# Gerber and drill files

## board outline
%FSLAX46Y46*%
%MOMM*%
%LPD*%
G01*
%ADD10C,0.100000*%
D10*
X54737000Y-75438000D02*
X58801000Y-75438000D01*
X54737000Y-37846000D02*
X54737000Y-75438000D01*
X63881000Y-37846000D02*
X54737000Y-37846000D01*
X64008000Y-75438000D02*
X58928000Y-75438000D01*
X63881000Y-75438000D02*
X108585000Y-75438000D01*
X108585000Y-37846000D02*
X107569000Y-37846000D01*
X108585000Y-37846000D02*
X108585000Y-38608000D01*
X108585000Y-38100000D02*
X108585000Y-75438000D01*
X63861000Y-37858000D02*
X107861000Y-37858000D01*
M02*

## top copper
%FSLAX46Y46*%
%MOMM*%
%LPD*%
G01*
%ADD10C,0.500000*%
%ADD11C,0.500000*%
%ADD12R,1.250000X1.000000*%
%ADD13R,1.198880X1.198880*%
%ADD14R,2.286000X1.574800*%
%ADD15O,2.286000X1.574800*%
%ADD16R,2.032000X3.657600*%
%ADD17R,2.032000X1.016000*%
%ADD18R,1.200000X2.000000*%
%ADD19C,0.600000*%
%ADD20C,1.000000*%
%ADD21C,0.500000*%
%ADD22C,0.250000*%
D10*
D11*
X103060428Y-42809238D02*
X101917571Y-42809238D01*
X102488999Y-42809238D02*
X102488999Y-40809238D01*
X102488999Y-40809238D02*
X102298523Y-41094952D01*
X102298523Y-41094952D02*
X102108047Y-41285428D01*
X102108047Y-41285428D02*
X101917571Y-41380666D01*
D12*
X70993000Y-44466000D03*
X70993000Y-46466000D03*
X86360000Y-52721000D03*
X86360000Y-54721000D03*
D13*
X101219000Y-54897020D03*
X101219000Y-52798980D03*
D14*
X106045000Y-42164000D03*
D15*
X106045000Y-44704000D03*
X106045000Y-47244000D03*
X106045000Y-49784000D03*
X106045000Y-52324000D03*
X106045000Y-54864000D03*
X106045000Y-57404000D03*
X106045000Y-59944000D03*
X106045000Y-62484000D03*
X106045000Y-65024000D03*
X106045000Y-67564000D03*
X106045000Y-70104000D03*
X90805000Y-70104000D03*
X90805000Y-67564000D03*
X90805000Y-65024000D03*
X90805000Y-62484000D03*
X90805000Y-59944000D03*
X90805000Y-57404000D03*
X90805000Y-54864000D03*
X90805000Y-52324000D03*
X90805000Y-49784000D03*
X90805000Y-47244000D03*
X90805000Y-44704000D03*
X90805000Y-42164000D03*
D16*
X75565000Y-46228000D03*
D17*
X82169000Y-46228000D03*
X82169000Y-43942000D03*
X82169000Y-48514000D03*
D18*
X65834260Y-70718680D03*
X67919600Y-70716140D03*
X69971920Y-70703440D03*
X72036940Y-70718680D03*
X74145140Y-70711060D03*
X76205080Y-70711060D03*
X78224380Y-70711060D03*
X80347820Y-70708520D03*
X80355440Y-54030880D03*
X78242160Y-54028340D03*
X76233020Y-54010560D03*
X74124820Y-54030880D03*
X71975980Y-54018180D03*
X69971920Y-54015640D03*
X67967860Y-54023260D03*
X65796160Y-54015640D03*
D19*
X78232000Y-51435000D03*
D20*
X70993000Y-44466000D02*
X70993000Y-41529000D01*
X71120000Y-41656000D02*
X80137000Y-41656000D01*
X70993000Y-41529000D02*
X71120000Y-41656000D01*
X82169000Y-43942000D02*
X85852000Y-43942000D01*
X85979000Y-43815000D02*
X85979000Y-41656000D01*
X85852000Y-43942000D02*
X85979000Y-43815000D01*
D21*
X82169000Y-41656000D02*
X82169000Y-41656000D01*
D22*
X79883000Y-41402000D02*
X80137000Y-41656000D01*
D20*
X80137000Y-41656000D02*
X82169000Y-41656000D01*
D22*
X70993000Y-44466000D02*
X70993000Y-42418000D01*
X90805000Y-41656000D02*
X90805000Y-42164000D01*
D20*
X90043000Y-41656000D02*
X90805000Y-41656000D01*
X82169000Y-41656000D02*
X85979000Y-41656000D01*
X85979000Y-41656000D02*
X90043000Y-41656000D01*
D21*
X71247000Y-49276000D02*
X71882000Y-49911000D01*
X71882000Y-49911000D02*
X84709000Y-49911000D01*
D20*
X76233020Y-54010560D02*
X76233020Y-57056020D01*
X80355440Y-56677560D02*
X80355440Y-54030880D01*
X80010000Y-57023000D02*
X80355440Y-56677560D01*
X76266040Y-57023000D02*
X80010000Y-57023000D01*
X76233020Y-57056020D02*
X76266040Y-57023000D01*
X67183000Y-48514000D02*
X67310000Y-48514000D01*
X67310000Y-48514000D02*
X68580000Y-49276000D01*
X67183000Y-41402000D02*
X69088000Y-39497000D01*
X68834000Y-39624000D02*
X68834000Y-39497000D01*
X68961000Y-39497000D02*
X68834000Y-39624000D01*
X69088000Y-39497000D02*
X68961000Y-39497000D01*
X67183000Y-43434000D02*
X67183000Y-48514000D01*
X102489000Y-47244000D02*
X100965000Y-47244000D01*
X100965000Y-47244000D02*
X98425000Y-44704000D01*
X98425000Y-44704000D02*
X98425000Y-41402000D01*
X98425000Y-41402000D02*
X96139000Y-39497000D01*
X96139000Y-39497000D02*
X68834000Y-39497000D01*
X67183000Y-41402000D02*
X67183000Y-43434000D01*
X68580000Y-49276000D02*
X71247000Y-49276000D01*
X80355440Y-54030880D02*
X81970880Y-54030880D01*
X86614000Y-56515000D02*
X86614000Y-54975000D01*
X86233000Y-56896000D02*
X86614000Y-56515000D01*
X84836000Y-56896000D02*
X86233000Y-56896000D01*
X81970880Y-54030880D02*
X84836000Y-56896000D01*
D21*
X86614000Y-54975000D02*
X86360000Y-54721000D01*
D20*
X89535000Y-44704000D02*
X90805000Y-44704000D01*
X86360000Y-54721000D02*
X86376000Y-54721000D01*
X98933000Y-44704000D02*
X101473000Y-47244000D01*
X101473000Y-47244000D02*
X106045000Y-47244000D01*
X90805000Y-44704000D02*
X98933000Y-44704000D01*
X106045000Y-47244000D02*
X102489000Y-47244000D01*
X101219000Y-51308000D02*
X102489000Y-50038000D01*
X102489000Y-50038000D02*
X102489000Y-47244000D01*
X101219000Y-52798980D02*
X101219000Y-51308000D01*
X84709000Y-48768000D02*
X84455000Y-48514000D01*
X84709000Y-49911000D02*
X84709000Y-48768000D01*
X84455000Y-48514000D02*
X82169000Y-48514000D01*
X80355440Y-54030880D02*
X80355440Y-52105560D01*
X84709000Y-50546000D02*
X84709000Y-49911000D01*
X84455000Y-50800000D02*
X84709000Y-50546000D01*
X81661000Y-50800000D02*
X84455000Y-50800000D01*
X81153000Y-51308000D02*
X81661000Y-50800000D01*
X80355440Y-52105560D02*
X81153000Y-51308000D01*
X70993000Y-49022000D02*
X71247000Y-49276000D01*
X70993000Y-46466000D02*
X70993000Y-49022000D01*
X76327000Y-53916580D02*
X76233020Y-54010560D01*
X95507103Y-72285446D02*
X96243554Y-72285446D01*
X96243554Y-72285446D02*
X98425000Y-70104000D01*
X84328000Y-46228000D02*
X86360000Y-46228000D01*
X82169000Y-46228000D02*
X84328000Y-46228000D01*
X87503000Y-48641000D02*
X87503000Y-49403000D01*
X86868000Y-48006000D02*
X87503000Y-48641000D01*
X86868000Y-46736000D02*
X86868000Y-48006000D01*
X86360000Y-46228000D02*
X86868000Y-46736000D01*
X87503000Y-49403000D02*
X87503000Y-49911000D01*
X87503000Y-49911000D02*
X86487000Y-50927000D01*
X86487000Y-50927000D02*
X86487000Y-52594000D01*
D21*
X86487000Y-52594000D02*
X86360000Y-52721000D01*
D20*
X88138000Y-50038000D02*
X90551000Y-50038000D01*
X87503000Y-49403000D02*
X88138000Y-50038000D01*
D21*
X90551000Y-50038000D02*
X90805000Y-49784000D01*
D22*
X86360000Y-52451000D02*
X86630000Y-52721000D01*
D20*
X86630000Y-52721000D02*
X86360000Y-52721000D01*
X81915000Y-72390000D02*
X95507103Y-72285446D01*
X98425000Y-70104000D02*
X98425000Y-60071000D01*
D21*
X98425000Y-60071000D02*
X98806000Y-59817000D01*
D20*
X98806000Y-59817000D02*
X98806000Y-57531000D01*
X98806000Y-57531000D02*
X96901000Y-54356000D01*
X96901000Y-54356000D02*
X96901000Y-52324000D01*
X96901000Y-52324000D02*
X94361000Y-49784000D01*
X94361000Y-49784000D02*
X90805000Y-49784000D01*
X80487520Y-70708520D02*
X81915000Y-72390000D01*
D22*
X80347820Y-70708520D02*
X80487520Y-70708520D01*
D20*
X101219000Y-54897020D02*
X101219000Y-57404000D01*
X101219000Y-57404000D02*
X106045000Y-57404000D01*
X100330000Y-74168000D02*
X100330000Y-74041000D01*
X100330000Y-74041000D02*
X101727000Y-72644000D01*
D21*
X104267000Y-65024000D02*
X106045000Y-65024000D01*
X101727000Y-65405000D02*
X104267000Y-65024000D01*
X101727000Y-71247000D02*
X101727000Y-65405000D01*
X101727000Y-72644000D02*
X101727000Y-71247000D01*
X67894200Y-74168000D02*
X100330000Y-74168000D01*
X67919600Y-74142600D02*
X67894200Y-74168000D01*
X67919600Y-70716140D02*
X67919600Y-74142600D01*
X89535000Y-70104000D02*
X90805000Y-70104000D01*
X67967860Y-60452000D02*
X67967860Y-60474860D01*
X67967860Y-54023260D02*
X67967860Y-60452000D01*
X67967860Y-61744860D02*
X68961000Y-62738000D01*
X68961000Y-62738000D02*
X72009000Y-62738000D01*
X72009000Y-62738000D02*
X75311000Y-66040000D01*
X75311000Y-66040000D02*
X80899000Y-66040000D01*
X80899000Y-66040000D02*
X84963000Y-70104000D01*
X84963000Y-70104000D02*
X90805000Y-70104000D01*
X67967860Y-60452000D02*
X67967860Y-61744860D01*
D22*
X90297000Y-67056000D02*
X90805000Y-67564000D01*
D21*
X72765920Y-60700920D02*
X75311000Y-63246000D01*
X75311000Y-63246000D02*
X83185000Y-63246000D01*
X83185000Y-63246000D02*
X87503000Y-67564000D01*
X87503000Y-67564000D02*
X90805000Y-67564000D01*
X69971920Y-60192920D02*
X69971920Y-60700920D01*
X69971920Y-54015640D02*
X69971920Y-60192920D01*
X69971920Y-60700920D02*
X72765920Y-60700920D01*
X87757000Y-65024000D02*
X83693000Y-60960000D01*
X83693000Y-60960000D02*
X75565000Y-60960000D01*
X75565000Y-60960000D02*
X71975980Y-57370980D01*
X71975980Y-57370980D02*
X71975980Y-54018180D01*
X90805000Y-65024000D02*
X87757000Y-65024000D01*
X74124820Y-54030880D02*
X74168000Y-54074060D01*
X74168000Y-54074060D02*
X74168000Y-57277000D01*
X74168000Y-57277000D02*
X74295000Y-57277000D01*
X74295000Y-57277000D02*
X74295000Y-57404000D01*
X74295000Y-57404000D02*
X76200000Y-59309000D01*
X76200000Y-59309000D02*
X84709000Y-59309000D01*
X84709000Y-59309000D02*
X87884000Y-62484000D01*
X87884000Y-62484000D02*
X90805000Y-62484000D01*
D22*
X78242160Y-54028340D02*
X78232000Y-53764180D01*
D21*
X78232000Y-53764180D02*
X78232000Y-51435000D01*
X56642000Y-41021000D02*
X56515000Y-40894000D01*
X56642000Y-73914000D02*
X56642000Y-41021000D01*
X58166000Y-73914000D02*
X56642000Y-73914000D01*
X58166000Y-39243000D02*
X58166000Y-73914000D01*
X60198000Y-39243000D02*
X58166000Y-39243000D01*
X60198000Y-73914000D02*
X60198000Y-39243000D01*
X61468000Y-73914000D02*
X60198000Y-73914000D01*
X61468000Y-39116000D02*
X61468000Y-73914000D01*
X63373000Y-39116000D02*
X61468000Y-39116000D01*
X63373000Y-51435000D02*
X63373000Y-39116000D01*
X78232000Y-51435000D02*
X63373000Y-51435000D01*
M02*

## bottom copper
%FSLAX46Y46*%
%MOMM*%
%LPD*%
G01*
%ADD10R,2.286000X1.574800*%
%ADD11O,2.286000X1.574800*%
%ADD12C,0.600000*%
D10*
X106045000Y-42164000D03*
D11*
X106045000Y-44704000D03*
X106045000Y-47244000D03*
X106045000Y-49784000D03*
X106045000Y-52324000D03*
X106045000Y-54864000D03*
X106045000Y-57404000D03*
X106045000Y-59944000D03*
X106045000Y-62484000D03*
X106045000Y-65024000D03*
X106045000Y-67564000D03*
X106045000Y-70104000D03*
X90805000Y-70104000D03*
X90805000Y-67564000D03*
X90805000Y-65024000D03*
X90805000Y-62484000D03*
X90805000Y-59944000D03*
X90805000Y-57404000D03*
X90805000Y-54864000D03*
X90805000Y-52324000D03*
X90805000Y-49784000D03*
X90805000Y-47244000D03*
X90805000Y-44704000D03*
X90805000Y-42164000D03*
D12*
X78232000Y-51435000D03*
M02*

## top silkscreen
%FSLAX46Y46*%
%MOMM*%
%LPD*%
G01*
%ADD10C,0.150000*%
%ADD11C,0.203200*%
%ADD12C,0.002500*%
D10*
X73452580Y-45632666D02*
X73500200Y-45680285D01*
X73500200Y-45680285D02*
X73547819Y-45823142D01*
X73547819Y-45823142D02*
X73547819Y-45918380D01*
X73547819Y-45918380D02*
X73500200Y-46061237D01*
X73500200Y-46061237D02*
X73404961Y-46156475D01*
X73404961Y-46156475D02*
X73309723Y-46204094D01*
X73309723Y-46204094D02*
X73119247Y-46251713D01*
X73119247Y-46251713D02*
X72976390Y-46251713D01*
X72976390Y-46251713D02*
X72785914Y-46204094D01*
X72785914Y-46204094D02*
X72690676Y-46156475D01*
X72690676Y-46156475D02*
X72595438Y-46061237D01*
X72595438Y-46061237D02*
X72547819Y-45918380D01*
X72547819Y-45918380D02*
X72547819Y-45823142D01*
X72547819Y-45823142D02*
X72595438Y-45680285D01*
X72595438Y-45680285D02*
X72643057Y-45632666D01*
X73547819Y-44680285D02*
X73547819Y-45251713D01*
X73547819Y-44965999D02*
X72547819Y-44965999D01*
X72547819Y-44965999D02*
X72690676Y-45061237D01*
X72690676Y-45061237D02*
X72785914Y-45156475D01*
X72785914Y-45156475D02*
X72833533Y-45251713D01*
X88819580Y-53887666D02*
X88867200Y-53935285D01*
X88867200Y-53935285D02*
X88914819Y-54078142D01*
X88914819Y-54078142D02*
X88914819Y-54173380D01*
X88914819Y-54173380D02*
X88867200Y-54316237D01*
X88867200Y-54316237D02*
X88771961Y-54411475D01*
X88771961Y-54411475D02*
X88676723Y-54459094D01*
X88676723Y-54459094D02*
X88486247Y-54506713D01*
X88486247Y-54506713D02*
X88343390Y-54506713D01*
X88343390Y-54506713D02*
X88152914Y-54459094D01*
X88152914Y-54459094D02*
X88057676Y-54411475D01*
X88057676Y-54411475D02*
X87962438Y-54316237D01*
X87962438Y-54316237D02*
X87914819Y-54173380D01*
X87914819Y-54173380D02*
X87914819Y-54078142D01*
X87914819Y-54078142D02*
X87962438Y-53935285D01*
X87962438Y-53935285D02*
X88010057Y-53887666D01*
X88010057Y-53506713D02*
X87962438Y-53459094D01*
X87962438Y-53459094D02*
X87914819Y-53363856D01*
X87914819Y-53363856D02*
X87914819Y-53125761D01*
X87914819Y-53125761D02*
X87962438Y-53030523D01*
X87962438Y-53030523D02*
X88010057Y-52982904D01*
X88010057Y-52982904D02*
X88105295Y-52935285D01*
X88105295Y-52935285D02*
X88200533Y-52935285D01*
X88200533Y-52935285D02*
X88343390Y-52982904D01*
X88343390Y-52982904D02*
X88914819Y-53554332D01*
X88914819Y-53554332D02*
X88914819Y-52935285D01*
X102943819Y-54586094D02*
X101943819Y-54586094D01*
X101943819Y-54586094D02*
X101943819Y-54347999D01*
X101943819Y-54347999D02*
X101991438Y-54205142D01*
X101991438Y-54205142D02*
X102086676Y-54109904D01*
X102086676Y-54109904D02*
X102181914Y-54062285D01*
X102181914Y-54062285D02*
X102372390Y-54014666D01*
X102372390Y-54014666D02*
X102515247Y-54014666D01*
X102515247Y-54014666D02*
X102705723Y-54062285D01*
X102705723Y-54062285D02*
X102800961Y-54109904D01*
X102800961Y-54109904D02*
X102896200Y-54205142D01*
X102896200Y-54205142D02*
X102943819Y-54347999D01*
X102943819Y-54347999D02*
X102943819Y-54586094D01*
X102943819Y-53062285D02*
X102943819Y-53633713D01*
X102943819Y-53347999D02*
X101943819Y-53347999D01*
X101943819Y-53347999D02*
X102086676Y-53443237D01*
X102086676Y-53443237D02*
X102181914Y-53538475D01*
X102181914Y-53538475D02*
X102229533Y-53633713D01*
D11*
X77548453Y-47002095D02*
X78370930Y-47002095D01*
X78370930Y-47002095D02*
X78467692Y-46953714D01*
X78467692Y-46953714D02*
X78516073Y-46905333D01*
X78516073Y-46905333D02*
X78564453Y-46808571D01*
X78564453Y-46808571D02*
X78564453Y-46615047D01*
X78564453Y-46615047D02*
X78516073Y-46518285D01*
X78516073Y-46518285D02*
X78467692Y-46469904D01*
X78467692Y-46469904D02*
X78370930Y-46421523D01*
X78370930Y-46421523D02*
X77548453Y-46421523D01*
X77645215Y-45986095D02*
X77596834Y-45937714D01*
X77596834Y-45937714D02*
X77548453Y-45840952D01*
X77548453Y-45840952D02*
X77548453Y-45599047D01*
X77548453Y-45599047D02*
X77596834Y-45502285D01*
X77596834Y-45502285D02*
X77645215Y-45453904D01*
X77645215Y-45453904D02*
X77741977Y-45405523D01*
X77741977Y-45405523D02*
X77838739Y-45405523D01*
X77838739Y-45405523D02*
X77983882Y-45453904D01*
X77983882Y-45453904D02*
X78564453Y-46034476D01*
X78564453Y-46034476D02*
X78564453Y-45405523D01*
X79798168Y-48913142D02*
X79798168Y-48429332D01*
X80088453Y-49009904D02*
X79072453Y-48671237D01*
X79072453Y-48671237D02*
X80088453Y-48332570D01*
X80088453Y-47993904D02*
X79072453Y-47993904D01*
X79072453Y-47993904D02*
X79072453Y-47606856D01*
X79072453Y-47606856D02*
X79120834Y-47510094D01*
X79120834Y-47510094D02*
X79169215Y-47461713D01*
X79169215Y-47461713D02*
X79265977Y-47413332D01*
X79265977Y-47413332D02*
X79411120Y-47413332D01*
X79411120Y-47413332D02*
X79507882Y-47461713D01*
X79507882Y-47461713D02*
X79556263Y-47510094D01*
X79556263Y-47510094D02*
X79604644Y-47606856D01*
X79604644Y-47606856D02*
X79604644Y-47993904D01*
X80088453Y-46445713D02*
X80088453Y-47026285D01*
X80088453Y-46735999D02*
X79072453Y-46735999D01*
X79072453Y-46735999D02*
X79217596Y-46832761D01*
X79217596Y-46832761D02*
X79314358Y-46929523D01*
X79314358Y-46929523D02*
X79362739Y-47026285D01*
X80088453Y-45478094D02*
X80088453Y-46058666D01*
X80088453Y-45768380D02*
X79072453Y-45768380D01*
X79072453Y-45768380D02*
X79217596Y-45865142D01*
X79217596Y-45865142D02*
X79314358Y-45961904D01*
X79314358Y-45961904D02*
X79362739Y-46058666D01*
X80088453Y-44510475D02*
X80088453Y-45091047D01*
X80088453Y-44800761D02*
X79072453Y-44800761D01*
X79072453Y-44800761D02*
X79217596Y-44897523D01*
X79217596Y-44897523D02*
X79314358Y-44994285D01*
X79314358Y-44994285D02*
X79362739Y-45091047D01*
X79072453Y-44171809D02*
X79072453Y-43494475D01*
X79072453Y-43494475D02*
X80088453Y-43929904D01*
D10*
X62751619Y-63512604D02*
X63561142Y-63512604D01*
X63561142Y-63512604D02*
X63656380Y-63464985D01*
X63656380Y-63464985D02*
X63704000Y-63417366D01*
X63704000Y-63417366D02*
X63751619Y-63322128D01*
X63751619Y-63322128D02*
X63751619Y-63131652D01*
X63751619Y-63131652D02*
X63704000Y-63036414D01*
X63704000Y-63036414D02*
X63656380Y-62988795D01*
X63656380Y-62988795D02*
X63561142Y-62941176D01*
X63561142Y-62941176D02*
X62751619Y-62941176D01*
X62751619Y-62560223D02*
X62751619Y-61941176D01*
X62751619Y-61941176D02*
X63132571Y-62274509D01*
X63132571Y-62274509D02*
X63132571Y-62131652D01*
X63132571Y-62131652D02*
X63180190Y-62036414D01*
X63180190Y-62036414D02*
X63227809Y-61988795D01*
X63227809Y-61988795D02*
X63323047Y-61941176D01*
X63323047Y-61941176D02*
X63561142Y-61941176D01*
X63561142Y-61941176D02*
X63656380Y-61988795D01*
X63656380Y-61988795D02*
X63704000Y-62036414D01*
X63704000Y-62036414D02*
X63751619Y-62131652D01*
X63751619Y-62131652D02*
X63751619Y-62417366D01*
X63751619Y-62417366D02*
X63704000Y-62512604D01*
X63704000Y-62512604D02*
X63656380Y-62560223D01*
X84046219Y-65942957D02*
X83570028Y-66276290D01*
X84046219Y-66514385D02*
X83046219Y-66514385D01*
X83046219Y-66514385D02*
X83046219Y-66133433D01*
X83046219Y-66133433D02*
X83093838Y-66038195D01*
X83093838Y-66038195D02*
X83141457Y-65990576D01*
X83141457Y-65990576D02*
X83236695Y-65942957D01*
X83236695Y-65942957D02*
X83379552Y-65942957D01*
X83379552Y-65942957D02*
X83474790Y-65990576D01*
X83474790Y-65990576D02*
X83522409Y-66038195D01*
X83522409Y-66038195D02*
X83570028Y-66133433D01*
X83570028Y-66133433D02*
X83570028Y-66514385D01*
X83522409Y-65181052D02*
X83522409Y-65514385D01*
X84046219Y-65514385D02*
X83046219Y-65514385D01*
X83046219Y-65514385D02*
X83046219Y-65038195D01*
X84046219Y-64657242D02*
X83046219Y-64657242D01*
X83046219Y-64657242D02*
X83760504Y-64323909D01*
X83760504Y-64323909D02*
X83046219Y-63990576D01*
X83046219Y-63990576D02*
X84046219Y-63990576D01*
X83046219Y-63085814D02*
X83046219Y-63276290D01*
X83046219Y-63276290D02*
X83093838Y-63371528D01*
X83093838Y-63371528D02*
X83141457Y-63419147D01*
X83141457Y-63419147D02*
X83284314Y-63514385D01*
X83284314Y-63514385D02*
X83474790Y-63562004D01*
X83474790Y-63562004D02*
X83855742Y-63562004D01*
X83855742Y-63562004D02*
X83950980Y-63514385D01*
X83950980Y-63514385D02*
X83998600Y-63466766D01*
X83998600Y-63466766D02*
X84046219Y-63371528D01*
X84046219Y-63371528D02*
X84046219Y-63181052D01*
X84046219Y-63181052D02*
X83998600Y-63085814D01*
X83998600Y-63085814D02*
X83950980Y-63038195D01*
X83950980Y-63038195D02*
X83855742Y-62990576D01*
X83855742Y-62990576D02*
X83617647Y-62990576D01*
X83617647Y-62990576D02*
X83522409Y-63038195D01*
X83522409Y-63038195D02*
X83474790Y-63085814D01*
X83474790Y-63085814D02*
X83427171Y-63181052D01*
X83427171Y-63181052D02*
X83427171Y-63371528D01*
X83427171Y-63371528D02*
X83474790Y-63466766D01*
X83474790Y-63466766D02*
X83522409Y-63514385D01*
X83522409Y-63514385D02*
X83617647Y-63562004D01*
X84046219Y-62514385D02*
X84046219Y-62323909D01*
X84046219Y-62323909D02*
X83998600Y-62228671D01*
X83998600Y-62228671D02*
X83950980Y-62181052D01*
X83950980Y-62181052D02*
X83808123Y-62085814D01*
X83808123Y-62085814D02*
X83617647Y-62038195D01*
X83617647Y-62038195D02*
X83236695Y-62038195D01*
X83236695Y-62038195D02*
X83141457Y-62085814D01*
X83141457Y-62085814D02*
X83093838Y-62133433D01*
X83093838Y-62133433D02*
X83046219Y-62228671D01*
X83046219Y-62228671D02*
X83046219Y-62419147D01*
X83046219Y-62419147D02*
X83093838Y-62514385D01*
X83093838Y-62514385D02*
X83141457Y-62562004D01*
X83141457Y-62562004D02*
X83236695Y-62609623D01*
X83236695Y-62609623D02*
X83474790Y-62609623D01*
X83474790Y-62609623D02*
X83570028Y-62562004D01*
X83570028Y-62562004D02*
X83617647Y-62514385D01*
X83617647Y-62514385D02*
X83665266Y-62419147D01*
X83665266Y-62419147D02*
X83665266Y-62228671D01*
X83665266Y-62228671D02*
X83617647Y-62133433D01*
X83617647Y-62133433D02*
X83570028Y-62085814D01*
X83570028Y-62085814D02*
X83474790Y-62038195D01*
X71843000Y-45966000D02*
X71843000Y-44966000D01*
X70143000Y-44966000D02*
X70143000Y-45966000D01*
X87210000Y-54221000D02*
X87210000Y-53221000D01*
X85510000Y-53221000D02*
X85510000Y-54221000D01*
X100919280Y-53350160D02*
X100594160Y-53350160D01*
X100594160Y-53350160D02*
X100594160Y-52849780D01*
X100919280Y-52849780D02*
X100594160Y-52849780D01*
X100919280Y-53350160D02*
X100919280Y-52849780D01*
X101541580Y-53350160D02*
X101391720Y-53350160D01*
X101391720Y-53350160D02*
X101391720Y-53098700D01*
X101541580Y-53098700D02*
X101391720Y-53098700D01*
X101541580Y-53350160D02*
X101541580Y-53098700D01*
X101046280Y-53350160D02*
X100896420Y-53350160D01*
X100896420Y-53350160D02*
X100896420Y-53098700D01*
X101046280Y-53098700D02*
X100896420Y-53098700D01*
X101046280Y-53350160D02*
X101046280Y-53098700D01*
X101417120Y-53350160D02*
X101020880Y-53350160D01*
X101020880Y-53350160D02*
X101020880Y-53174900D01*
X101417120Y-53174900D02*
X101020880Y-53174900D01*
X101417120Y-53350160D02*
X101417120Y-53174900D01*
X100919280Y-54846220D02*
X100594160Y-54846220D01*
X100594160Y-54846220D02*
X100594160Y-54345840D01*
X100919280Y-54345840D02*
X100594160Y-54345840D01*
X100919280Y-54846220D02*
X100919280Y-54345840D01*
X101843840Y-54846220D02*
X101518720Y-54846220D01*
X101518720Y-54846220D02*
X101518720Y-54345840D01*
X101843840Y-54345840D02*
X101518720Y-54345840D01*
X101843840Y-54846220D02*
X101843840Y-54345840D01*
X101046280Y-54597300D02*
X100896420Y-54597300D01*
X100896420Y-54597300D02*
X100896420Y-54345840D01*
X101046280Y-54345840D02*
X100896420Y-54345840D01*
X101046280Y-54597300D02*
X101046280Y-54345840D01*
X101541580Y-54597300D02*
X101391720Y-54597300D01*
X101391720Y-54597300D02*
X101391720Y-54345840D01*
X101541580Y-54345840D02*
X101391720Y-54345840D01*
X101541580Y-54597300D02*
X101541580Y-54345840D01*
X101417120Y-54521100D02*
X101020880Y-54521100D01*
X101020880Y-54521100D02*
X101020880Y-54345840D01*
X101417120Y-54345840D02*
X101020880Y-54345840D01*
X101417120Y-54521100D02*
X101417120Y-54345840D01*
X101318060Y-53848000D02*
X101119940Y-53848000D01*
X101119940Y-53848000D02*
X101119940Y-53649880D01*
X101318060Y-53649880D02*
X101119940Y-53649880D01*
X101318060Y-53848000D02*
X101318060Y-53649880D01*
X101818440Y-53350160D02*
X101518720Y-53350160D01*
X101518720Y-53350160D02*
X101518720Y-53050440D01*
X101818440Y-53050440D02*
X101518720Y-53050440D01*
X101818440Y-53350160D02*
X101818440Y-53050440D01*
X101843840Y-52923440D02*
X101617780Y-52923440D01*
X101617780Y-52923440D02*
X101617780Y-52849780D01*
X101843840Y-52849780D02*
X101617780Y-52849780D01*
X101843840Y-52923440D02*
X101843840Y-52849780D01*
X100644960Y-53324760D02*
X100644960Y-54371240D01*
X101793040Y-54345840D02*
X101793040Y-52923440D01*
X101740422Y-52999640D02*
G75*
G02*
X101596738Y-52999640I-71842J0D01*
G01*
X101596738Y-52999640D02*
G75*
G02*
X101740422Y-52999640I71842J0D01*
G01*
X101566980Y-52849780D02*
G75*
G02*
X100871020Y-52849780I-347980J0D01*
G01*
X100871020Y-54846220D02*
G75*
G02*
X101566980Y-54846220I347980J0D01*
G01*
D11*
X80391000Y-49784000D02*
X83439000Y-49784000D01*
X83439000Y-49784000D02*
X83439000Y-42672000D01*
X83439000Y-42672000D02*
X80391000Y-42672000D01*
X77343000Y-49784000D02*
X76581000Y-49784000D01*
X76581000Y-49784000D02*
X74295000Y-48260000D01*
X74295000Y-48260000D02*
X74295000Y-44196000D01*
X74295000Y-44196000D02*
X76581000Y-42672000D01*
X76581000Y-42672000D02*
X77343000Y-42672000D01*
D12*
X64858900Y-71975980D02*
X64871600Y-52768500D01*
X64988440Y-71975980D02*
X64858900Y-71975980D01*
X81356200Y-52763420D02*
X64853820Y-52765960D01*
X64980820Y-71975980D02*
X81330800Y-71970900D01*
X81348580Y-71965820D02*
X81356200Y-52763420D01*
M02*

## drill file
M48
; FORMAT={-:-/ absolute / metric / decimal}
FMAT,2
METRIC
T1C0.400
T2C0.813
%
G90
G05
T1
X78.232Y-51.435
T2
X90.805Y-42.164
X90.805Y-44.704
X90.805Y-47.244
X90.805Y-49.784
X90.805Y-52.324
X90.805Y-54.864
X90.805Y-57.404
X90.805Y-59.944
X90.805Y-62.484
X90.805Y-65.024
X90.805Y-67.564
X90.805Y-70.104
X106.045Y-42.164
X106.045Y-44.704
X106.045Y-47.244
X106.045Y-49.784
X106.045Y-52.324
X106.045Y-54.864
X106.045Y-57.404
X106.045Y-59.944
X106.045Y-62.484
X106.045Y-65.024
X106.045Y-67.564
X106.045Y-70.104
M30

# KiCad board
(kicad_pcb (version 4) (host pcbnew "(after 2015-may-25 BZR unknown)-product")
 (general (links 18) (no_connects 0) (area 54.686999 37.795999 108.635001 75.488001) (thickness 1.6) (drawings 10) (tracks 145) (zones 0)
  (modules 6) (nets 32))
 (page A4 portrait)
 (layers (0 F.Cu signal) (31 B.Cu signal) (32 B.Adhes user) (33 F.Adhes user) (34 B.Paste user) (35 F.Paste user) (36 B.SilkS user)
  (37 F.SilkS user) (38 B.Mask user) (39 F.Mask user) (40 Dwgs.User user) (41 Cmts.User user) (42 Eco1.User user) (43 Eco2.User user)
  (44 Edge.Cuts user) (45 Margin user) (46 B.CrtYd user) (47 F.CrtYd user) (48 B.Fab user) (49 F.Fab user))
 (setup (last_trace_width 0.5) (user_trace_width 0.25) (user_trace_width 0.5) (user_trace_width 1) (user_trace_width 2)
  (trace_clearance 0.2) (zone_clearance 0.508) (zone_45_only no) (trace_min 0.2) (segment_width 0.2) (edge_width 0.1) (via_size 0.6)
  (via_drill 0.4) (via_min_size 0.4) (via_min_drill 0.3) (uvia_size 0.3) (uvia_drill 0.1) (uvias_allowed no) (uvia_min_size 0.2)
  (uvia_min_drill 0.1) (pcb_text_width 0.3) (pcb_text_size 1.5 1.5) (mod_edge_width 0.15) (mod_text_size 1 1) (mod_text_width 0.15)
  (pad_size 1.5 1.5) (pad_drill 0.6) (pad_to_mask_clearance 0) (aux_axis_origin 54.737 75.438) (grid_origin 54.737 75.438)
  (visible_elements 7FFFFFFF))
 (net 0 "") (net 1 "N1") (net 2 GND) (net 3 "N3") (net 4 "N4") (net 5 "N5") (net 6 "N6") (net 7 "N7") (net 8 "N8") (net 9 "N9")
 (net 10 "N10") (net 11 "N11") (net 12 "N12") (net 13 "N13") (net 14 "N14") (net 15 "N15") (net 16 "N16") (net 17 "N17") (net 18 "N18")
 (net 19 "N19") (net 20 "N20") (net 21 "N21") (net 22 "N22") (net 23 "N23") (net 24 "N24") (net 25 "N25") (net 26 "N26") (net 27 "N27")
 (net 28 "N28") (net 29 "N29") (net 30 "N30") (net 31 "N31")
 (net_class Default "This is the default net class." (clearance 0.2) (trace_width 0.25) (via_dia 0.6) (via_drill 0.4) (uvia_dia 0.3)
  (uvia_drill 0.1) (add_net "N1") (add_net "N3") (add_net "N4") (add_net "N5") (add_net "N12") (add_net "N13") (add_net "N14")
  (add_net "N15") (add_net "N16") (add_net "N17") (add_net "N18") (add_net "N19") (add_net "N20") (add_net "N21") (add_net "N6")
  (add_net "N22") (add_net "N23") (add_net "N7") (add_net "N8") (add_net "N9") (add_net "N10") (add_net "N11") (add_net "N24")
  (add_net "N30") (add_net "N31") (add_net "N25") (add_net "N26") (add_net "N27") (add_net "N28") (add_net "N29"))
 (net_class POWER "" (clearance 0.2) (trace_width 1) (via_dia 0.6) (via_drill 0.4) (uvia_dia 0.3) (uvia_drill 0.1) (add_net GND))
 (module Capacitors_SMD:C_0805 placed (layer F.Cu) (at 70.993 45.466 270)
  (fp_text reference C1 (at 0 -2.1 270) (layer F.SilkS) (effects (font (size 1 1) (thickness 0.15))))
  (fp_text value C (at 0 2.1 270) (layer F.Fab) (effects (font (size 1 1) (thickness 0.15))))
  (fp_line (start 0.5 -0.85) (end -0.5 -0.85) (layer F.SilkS) (width 0.15))
  (fp_line (start -0.5 0.85) (end 0.5 0.85) (layer F.SilkS) (width 0.15))
  (pad 1 smd rect (at -1 0 270) (size 1 1.25) (layers F.Cu F.Paste F.Mask) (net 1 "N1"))
  (pad 2 smd rect (at 1 0 270) (size 1 1.25) (layers F.Cu F.Paste F.Mask) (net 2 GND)))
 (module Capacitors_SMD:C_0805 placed (layer F.Cu) (at 86.36 53.721 270)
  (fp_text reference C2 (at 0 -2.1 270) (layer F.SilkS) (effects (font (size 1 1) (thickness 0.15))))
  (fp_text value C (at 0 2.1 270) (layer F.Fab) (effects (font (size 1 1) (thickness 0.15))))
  (fp_line (start 0.5 -0.85) (end -0.5 -0.85) (layer F.SilkS) (width 0.15))
  (fp_line (start -0.5 0.85) (end 0.5 0.85) (layer F.SilkS) (width 0.15))
  (pad 1 smd rect (at -1 0 270) (size 1 1.25) (layers F.Cu F.Paste F.Mask) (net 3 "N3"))
  (pad 2 smd rect (at 1 0 270) (size 1 1.25) (layers F.Cu F.Paste F.Mask) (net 2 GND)))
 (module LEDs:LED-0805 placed (layer F.Cu) (at 101.219 53.848 270)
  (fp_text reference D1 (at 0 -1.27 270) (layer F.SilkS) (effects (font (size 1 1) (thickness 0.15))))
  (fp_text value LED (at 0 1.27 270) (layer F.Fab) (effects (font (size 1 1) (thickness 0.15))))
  (fp_line (start -0.49784 0.29972) (end -0.49784 0.62484) (layer F.SilkS) (width 0.15))
  (fp_line (start -0.49784 0.62484) (end -0.99822 0.62484) (layer F.SilkS) (width 0.15))
  (fp_line (start -0.99822 0.29972) (end -0.99822 0.62484) (layer F.SilkS) (width 0.15))
  (fp_line (start -0.49784 0.29972) (end -0.99822 0.29972) (layer F.SilkS) (width 0.15))
  (fp_line (start -0.49784 -0.32258) (end -0.49784 -0.17272) (layer F.SilkS) (width 0.15))
  (fp_line (start -0.49784 -0.17272) (end -0.7493 -0.17272) (layer F.SilkS) (width 0.15))
  (fp_line (start -0.7493 -0.32258) (end -0.7493 -0.17272) (layer F.SilkS) (width 0.15))
  (fp_line (start -0.49784 -0.32258) (end -0.7493 -0.32258) (layer F.SilkS) (width 0.15))
  (fp_line (start -0.49784 0.17272) (end -0.49784 0.32258) (layer F.SilkS) (width 0.15))
  (fp_line (start -0.49784 0.32258) (end -0.7493 0.32258) (layer F.SilkS) (width 0.15))
  (fp_line (start -0.7493 0.17272) (end -0.7493 0.32258) (layer F.SilkS) (width 0.15))
  (fp_line (start -0.49784 0.17272) (end -0.7493 0.17272) (layer F.SilkS) (width 0.15))
  (fp_line (start -0.49784 -0.19812) (end -0.49784 0.19812) (layer F.SilkS) (width 0.15))
  (fp_line (start -0.49784 0.19812) (end -0.6731 0.19812) (layer F.SilkS) (width 0.15))
  (fp_line (start -0.6731 -0.19812) (end -0.6731 0.19812) (layer F.SilkS) (width 0.15))
  (fp_line (start -0.49784 -0.19812) (end -0.6731 -0.19812) (layer F.SilkS) (width 0.15))
  (fp_line (start 0.99822 0.29972) (end 0.99822 0.62484) (layer F.SilkS) (width 0.15))
  (fp_line (start 0.99822 0.62484) (end 0.49784 0.62484) (layer F.SilkS) (width 0.15))
  (fp_line (start 0.49784 0.29972) (end 0.49784 0.62484) (layer F.SilkS) (width 0.15))
  (fp_line (start 0.99822 0.29972) (end 0.49784 0.29972) (layer F.SilkS) (width 0.15))
  (fp_line (start 0.99822 -0.62484) (end 0.99822 -0.29972) (layer F.SilkS) (width 0.15))
  (fp_line (start 0.99822 -0.29972) (end 0.49784 -0.29972) (layer F.SilkS) (width 0.15))
  (fp_line (start 0.49784 -0.62484) (end 0.49784 -0.29972) (layer F.SilkS) (width 0.15))
  (fp_line (start 0.99822 -0.62484) (end 0.49784 -0.62484) (layer F.SilkS) (width 0.15))
  (fp_line (start 0.7493 0.17272) (end 0.7493 0.32258) (layer F.SilkS) (width 0.15))
  (fp_line (start 0.7493 0.32258) (end 0.49784 0.32258) (layer F.SilkS) (width 0.15))
  (fp_line (start 0.49784 0.17272) (end 0.49784 0.32258) (layer F.SilkS) (width 0.15))
  (fp_line (start 0.7493 0.17272) (end 0.49784 0.17272) (layer F.SilkS) (width 0.15))
  (fp_line (start 0.7493 -0.32258) (end 0.7493 -0.17272) (layer F.SilkS) (width 0.15))
  (fp_line (start 0.7493 -0.17272) (end 0.49784 -0.17272) (layer F.SilkS) (width 0.15))
  (fp_line (start 0.49784 -0.32258) (end 0.49784 -0.17272) (layer F.SilkS) (width 0.15))
  (fp_line (start 0.7493 -0.32258) (end 0.49784 -0.32258) (layer F.SilkS) (width 0.15))
  (fp_line (start 0.6731 -0.19812) (end 0.6731 0.19812) (layer F.SilkS) (width 0.15))
  (fp_line (start 0.6731 0.19812) (end 0.49784 0.19812) (layer F.SilkS) (width 0.15))
  (fp_line (start 0.49784 -0.19812) (end 0.49784 0.19812) (layer F.SilkS) (width 0.15))
  (fp_line (start 0.6731 -0.19812) (end 0.49784 -0.19812) (layer F.SilkS) (width 0.15))
  (fp_line (start 0 -0.09906) (end 0 0.09906) (layer F.SilkS) (width 0.15))
  (fp_line (start 0 0.09906) (end -0.19812 0.09906) (layer F.SilkS) (width 0.15))
  (fp_line (start -0.19812 -0.09906) (end -0.19812 0.09906) (layer F.SilkS) (width 0.15))
  (fp_line (start 0 -0.09906) (end -0.19812 -0.09906) (layer F.SilkS) (width 0.15))
  (fp_line (start -0.49784 -0.59944) (end -0.49784 -0.29972) (layer F.SilkS) (width 0.15))
  (fp_line (start -0.49784 -0.29972) (end -0.79756 -0.29972) (layer F.SilkS) (width 0.15))
  (fp_line (start -0.79756 -0.59944) (end -0.79756 -0.29972) (layer F.SilkS) (width 0.15))
  (fp_line (start -0.49784 -0.59944) (end -0.79756 -0.59944) (layer F.SilkS) (width 0.15))
  (fp_line (start -0.92456 -0.62484) (end -0.92456 -0.39878) (layer F.SilkS) (width 0.15))
  (fp_line (start -0.92456 -0.39878) (end -0.99822 -0.39878) (layer F.SilkS) (width 0.15))
  (fp_line (start -0.99822 -0.62484) (end -0.99822 -0.39878) (layer F.SilkS) (width 0.15))
  (fp_line (start -0.92456 -0.62484) (end -0.99822 -0.62484) (layer F.SilkS) (width 0.15))
  (fp_line (start -0.52324 0.57404) (end 0.52324 0.57404) (layer F.SilkS) (width 0.15))
  (fp_line (start 0.49784 -0.57404) (end -0.92456 -0.57404) (layer F.SilkS) (width 0.15))
  (fp_circle (center -0.84836 -0.44958) (end -0.89916 -0.50038) (layer F.SilkS) (width 0.15))
  (fp_arc (start -0.99822 0) (end -0.99822 0.34798) (angle -180) (layer F.SilkS) (width 0.15))
  (fp_arc (start 0.99822 0) (end 0.99822 -0.34798) (angle -180) (layer F.SilkS) (width 0.15))
  (pad 2 smd rect (at 1.04902 0 90) (size 1.19888 1.19888) (layers F.Cu F.Paste F.Mask) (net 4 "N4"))
  (pad 1 smd rect (at -1.04902 0 90) (size 1.19888 1.19888) (layers F.Cu F.Paste F.Mask) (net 2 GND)))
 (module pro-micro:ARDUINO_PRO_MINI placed (layer B.Cu) (at 102.235 56.134 270)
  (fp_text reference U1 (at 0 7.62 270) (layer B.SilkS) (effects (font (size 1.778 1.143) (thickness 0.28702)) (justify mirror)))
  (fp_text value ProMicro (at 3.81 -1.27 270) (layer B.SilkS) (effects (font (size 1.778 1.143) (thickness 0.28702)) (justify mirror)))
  (pad 1 thru_hole rect (at -13.97 -3.81 270) (size 1.5748 2.286) (drill 0.8128) (layers *.Cu *.Mask B.SilkS) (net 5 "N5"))
  (pad 2 thru_hole oval (at -11.43 -3.81 270) (size 1.5748 2.286) (drill 0.8128) (layers *.Cu *.Mask B.SilkS) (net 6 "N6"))
  (pad 3 thru_hole oval (at -8.89 -3.81 270) (size 1.5748 2.286) (drill 0.8128) (layers *.Cu *.Mask B.SilkS) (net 2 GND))
  (pad 4 thru_hole oval (at -6.35 -3.81 270) (size 1.5748 2.286) (drill 0.8128) (layers *.Cu *.Mask B.SilkS) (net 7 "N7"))
  (pad 5 thru_hole oval (at -3.81 -3.81 270) (size 1.5748 2.286) (drill 0.8128) (layers *.Cu *.Mask B.SilkS) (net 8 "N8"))
  (pad 6 thru_hole oval (at -1.27 -3.81 270) (size 1.5748 2.286) (drill 0.8128) (layers *.Cu *.Mask B.SilkS) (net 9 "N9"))
  (pad 7 thru_hole oval (at 1.27 -3.81 270) (size 1.5748 2.286) (drill 0.8128) (layers *.Cu *.Mask B.SilkS) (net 4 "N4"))
  (pad 8 thru_hole oval (at 3.81 -3.81 270) (size 1.5748 2.286) (drill 0.8128) (layers *.Cu *.Mask B.SilkS) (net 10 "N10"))
  (pad 9 thru_hole oval (at 6.35 -3.81 270) (size 1.5748 2.286) (drill 0.8128) (layers *.Cu *.Mask B.SilkS) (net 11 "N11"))
  (pad 10 thru_hole oval (at 8.89 -3.81 270) (size 1.5748 2.286) (drill 0.8128) (layers *.Cu *.Mask B.SilkS) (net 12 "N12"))
  (pad 11 thru_hole oval (at 11.43 -3.81 270) (size 1.5748 2.286) (drill 0.8128) (layers *.Cu *.Mask B.SilkS) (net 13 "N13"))
  (pad 12 thru_hole oval (at 13.97 -3.81 270) (size 1.5748 2.286) (drill 0.8128) (layers *.Cu *.Mask B.SilkS) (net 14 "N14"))
  (pad 13 thru_hole oval (at 13.97 11.43 270) (size 1.5748 2.286) (drill 0.8128) (layers *.Cu *.Mask B.SilkS) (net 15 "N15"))
  (pad 14 thru_hole oval (at 11.43 11.43 270) (size 1.5748 2.286) (drill 0.8128) (layers *.Cu *.Mask B.SilkS) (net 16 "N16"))
  (pad 15 thru_hole oval (at 8.89 11.43 270) (size 1.5748 2.286) (drill 0.8128) (layers *.Cu *.Mask B.SilkS) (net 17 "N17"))
  (pad 16 thru_hole oval (at 6.35 11.43 270) (size 1.5748 2.286) (drill 0.8128) (layers *.Cu *.Mask B.SilkS) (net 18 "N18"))
  (pad 17 thru_hole oval (at 3.81 11.43 270) (size 1.5748 2.286) (drill 0.8128) (layers *.Cu *.Mask B.SilkS) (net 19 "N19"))
  (pad 18 thru_hole oval (at 1.27 11.43 270) (size 1.5748 2.286) (drill 0.8128) (layers *.Cu *.Mask B.SilkS) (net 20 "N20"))
  (pad 19 thru_hole oval (at -1.27 11.43 270) (size 1.5748 2.286) (drill 0.8128) (layers *.Cu *.Mask B.SilkS) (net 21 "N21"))
  (pad 20 thru_hole oval (at -3.81 11.43 270) (size 1.5748 2.286) (drill 0.8128) (layers *.Cu *.Mask B.SilkS) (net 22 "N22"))
  (pad 21 thru_hole oval (at -6.35 11.43 270) (size 1.5748 2.286) (drill 0.8128) (layers *.Cu *.Mask B.SilkS) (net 3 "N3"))
  (pad 22 thru_hole oval (at -8.89 11.43 270) (size 1.5748 2.286) (drill 0.8128) (layers *.Cu *.Mask B.SilkS) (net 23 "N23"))
  (pad 23 thru_hole oval (at -11.43 11.43 270) (size 1.5748 2.286) (drill 0.8128) (layers *.Cu *.Mask B.SilkS) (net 2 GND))
  (pad 24 thru_hole oval (at -13.97 11.43 270) (size 1.5748 2.286) (drill 0.8128) (layers *.Cu *.Mask B.SilkS) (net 1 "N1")))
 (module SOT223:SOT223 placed (layer F.Cu) (at 78.867 46.228 90)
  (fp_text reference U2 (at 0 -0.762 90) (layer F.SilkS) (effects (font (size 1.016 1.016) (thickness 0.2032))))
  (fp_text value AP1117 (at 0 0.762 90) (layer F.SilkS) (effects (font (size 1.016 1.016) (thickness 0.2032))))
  (fp_line (start -3.556 1.524) (end -3.556 4.572) (layer F.SilkS) (width 0.2032))
  (fp_line (start -3.556 4.572) (end 3.556 4.572) (layer F.SilkS) (width 0.2032))
  (fp_line (start 3.556 4.572) (end 3.556 1.524) (layer F.SilkS) (width 0.2032))
  (fp_line (start -3.556 -1.524) (end -3.556 -2.286) (layer F.SilkS) (width 0.2032))
  (fp_line (start -3.556 -2.286) (end -2.032 -4.572) (layer F.SilkS) (width 0.2032))
  (fp_line (start -2.032 -4.572) (end 2.032 -4.572) (layer F.SilkS) (width 0.2032))
  (fp_line (start 2.032 -4.572) (end 3.556 -2.286) (layer F.SilkS) (width 0.2032))
  (fp_line (start 3.556 -2.286) (end 3.556 -1.524) (layer F.SilkS) (width 0.2032))
  (pad 4 smd rect (at 0 -3.302 90) (size 3.6576 2.032) (layers F.Cu F.Paste F.Mask))
  (pad 2 smd rect (at 0 3.302 90) (size 1.016 2.032) (layers F.Cu F.Paste F.Mask) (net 3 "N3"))
  (pad 3 smd rect (at 2.286 3.302 90) (size 1.016 2.032) (layers F.Cu F.Paste F.Mask) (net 1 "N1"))
  (pad 1 smd rect (at -2.286 3.302 90) (size 1.016 2.032) (layers F.Cu F.Paste F.Mask) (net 2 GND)))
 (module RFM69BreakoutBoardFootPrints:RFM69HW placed (layer F.Cu) (at 74.041 62.738 90)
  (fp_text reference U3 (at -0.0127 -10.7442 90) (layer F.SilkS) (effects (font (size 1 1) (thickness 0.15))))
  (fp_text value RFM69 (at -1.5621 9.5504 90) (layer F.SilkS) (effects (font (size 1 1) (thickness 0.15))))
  (fp_line (start -9.23798 -9.1821) (end 9.9695 -9.1694) (layer F.SilkS) (width 0.0025))
  (fp_line (start -9.23798 -9.05256) (end -9.23798 -9.1821) (layer F.SilkS) (width 0.0025))
  (fp_line (start 9.97458 7.3152) (end 9.97204 -9.18718) (layer F.SilkS) (width 0.0025))
  (fp_line (start -9.23798 -9.06018) (end -9.2329 7.2898) (layer F.SilkS) (width 0.0025))
  (fp_line (start -9.22782 7.30758) (end 9.97458 7.3152) (layer F.SilkS) (width 0.0025))
  (pad 1 smd rect (at -7.98068 -8.20674 90) (size 2 1.2) (layers F.Cu F.Paste F.Mask) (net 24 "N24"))
  (pad 2 smd rect (at -7.97814 -6.1214 90) (size 2 1.2) (layers F.Cu F.Paste F.Mask) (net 12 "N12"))
  (pad 3 smd rect (at -7.96544 -4.06908 90) (size 2 1.2) (layers F.Cu F.Paste F.Mask) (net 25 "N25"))
  (pad 4 smd rect (at -7.98068 -2.00406 90) (size 2 1.2) (layers F.Cu F.Paste F.Mask) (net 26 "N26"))
  (pad 5 smd rect (at -7.97306 0.10414 90) (size 2 1.2) (layers F.Cu F.Paste F.Mask) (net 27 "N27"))
  (pad 6 smd rect (at -7.97306 2.16408 90) (size 2 1.2) (layers F.Cu F.Paste F.Mask) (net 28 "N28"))
  (pad 7 smd rect (at -7.97306 4.18338 90) (size 2 1.2) (layers F.Cu F.Paste F.Mask) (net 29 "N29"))
  (pad 8 smd rect (at -7.97052 6.30682 90) (size 2 1.2) (layers F.Cu F.Paste F.Mask) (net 3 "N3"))
  (pad 9 smd rect (at 8.70712 6.31444 90) (size 2 1.2) (layers F.Cu F.Paste F.Mask) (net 2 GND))
  (pad 10 smd rect (at 8.70966 4.20116 90) (size 2 1.2) (layers F.Cu F.Paste F.Mask) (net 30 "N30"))
  (pad 11 smd rect (at 8.72744 2.19202 90) (size 2 1.2) (layers F.Cu F.Paste F.Mask) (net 2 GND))
  (pad 12 smd rect (at 8.70712 0.08382 90) (size 2 1.2) (layers F.Cu F.Paste F.Mask) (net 18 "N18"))
  (pad 13 smd rect (at 8.71982 -2.06502 90) (size 2 1.2) (layers F.Cu F.Paste F.Mask) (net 17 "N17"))
  (pad 14 smd rect (at 8.72236 -4.06908 90) (size 2 1.2) (layers F.Cu F.Paste F.Mask) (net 16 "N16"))
  (pad 15 smd rect (at 8.71474 -6.07314 90) (size 2 1.2) (layers F.Cu F.Paste F.Mask) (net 15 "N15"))
  (pad 16 smd rect (at 8.72236 -8.24484 90) (size 2 1.2) (layers F.Cu F.Paste F.Mask) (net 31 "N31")))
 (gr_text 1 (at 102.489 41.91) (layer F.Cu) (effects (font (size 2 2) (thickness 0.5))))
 (gr_line (start 54.737 75.438) (end 58.801 75.438) (angle 90) (layer Edge.Cuts) (width 0.1))
 (gr_line (start 54.737 37.846) (end 54.737 75.438) (angle 90) (layer Edge.Cuts) (width 0.1))
 (gr_line (start 63.881 37.846) (end 54.737 37.846) (angle 90) (layer Edge.Cuts) (width 0.1))
 (gr_line (start 64.008 75.438) (end 58.928 75.438) (angle 90) (layer Edge.Cuts) (width 0.1))
 (gr_line (start 63.881 75.438) (end 108.585 75.438) (angle 90) (layer Edge.Cuts) (width 0.1))
 (gr_line (start 108.585 37.846) (end 107.569 37.846) (angle 90) (layer Edge.Cuts) (width 0.1))
 (gr_line (start 108.585 37.846) (end 108.585 38.608) (angle 90) (layer Edge.Cuts) (width 0.1))
 (gr_line (start 108.585 38.1) (end 108.585 75.438) (angle 90) (layer Edge.Cuts) (width 0.1))
 (gr_line (start 63.861 37.858) (end 107.861 37.858) (angle 90) (layer Edge.Cuts) (width 0.1))
 (segment (start 70.993 44.466) (end 70.993 41.529) (width 1) (layer F.Cu) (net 1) (status 10))
 (segment (start 71.12 41.656) (end 80.137 41.656) (width 1) (layer F.Cu) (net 1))
 (segment (start 70.993 41.529) (end 71.12 41.656) (width 1) (layer F.Cu) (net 1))
 (segment (start 82.169 43.942) (end 85.852 43.942) (width 1) (layer F.Cu) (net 1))
 (segment (start 85.979 43.815) (end 85.979 41.656) (width 1) (layer F.Cu) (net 1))
 (segment (start 85.852 43.942) (end 85.979 43.815) (width 1) (layer F.Cu) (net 1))
 (segment (start 82.169 41.656) (end 82.169 41.656) (width 0.5) (layer F.Cu) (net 1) (status 20))
 (segment (start 79.883 41.402) (end 80.137 41.656) (width 0.25) (layer F.Cu) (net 1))
 (segment (start 80.137 41.656) (end 82.169 41.656) (width 1) (layer F.Cu) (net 1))
 (segment (start 70.993 44.466) (end 70.993 42.418) (width 0.25) (layer F.Cu) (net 1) (status 10))
 (segment (start 90.805 41.656) (end 90.805 42.164) (width 0.25) (layer F.Cu) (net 1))
 (segment (start 90.043 41.656) (end 90.805 41.656) (width 1) (layer F.Cu) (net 1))
 (segment (start 82.169 41.656) (end 85.979 41.656) (width 1) (layer F.Cu) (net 1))
 (segment (start 85.979 41.656) (end 90.043 41.656) (width 1) (layer F.Cu) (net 1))
 (segment (start 71.247 49.276) (end 71.882 49.911) (width 0.5) (layer F.Cu) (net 2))
 (segment (start 71.882 49.911) (end 84.709 49.911) (width 0.5) (layer F.Cu) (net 2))
 (segment (start 76.23302 54.01056) (end 76.23302 57.05602) (width 1) (layer F.Cu) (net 2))
 (segment (start 80.35544 56.67756) (end 80.35544 54.03088) (width 1) (layer F.Cu) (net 2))
 (segment (start 80.01 57.023) (end 80.35544 56.67756) (width 1) (layer F.Cu) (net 2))
 (segment (start 76.26604 57.023) (end 80.01 57.023) (width 1) (layer F.Cu) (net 2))
 (segment (start 76.23302 57.05602) (end 76.26604 57.023) (width 1) (layer F.Cu) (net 2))
 (segment (start 67.183 48.514) (end 67.31 48.514) (width 1) (layer F.Cu) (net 2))
 (segment (start 67.31 48.514) (end 68.58 49.276) (width 1) (layer F.Cu) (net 2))
 (segment (start 67.183 41.402) (end 69.088 39.497) (width 1) (layer F.Cu) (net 2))
 (segment (start 68.834 39.624) (end 68.834 39.497) (width 1) (layer F.Cu) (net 2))
 (segment (start 68.961 39.497) (end 68.834 39.624) (width 1) (layer F.Cu) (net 2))
 (segment (start 69.088 39.497) (end 68.961 39.497) (width 1) (layer F.Cu) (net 2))
 (segment (start 67.183 43.434) (end 67.183 48.514) (width 1) (layer F.Cu) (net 2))
 (segment (start 102.489 47.244) (end 100.965 47.244) (width 1) (layer F.Cu) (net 2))
 (segment (start 100.965 47.244) (end 98.425 44.704) (width 1) (layer F.Cu) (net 2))
 (segment (start 98.425 44.704) (end 98.425 41.402) (width 1) (layer F.Cu) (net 2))
 (segment (start 98.425 41.402) (end 96.139 39.497) (width 1) (layer F.Cu) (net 2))
 (segment (start 96.139 39.497) (end 68.834 39.497) (width 1) (layer F.Cu) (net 2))
 (segment (start 67.183 41.402) (end 67.183 43.434) (width 1) (layer F.Cu) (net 2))
 (segment (start 68.58 49.276) (end 71.247 49.276) (width 1) (layer F.Cu) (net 2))
 (segment (start 80.35544 54.03088) (end 81.97088 54.03088) (width 1) (layer F.Cu) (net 2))
 (segment (start 86.614 56.515) (end 86.614 54.975) (width 1) (layer F.Cu) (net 2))
 (segment (start 86.233 56.896) (end 86.614 56.515) (width 1) (layer F.Cu) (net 2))
 (segment (start 84.836 56.896) (end 86.233 56.896) (width 1) (layer F.Cu) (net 2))
 (segment (start 81.97088 54.03088) (end 84.836 56.896) (width 1) (layer F.Cu) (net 2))
 (segment (start 86.614 54.975) (end 86.36 54.721) (width 0.5) (layer F.Cu) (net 2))
 (segment (start 89.535 44.704) (end 90.805 44.704) (width 1) (layer F.Cu) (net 2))
 (segment (start 86.36 54.721) (end 86.376 54.721) (width 1) (layer F.Cu) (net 2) (status 30))
 (segment (start 98.933 44.704) (end 101.473 47.244) (width 1) (layer F.Cu) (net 2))
 (segment (start 101.473 47.244) (end 106.045 47.244) (width 1) (layer F.Cu) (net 2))
 (segment (start 90.805 44.704) (end 98.933 44.704) (width 1) (layer F.Cu) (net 2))
 (segment (start 106.045 47.244) (end 102.489 47.244) (width 1) (layer F.Cu) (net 2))
 (segment (start 101.219 51.308) (end 102.489 50.038) (width 1) (layer F.Cu) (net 2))
 (segment (start 102.489 50.038) (end 102.489 47.244) (width 1) (layer F.Cu) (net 2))
 (segment (start 101.219 52.79898) (end 101.219 51.308) (width 1) (layer F.Cu) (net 2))
 (segment (start 84.709 48.768) (end 84.455 48.514) (width 1) (layer F.Cu) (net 2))
 (segment (start 84.709 49.911) (end 84.709 48.768) (width 1) (layer F.Cu) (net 2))
 (segment (start 84.455 48.514) (end 82.169 48.514) (width 1) (layer F.Cu) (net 2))
 (segment (start 80.35544 54.03088) (end 80.35544 52.10556) (width 1) (layer F.Cu) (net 2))
 (segment (start 84.709 50.546) (end 84.709 49.911) (width 1) (layer F.Cu) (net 2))
 (segment (start 84.455 50.8) (end 84.709 50.546) (width 1) (layer F.Cu) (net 2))
 (segment (start 81.661 50.8) (end 84.455 50.8) (width 1) (layer F.Cu) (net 2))
 (segment (start 81.153 51.308) (end 81.661 50.8) (width 1) (layer F.Cu) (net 2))
 (segment (start 80.35544 52.10556) (end 81.153 51.308) (width 1) (layer F.Cu) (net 2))
 (segment (start 70.993 49.022) (end 71.247 49.276) (width 1) (layer F.Cu) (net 2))
 (segment (start 70.993 46.466) (end 70.993 49.022) (width 1) (layer F.Cu) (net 2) (status 10))
 (segment (start 76.327 53.91658) (end 76.23302 54.01056) (width 1) (layer F.Cu) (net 2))
 (segment (start 95.507103 72.285446) (end 96.243554 72.285446) (width 1) (layer F.Cu) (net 3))
 (segment (start 96.243554 72.285446) (end 98.425 70.104) (width 1) (layer F.Cu) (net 3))
 (segment (start 84.328 46.228) (end 86.36 46.228) (width 1) (layer F.Cu) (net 3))
 (segment (start 82.169 46.228) (end 84.328 46.228) (width 1) (layer F.Cu) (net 3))
 (segment (start 87.503 48.641) (end 87.503 49.403) (width 1) (layer F.Cu) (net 3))
 (segment (start 86.868 48.006) (end 87.503 48.641) (width 1) (layer F.Cu) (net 3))
 (segment (start 86.868 46.736) (end 86.868 48.006) (width 1) (layer F.Cu) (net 3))
 (segment (start 86.36 46.228) (end 86.868 46.736) (width 1) (layer F.Cu) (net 3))
 (segment (start 87.503 49.403) (end 87.503 49.911) (width 1) (layer F.Cu) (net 3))
 (segment (start 87.503 49.911) (end 86.487 50.927) (width 1) (layer F.Cu) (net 3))
 (segment (start 86.487 50.927) (end 86.487 52.594) (width 1) (layer F.Cu) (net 3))
 (segment (start 86.487 52.594) (end 86.36 52.721) (width 0.5) (layer F.Cu) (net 3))
 (segment (start 88.138 50.038) (end 90.551 50.038) (width 1) (layer F.Cu) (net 3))
 (segment (start 87.503 49.403) (end 88.138 50.038) (width 1) (layer F.Cu) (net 3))
 (segment (start 90.551 50.038) (end 90.805 49.784) (width 0.5) (layer F.Cu) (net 3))
 (segment (start 86.36 52.451) (end 86.63 52.721) (width 0.25) (layer F.Cu) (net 3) (status 30))
 (segment (start 86.63 52.721) (end 86.36 52.721) (width 1) (layer F.Cu) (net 3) (status 30))
 (segment (start 81.915 72.39) (end 95.507103 72.285446) (width 1) (layer F.Cu) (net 3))
 (segment (start 98.425 70.104) (end 98.425 60.071) (width 1) (layer F.Cu) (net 3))
 (segment (start 98.425 60.071) (end 98.806 59.817) (width 0.5) (layer F.Cu) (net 3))
 (segment (start 98.806 59.817) (end 98.806 57.531) (width 1) (layer F.Cu) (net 3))
 (segment (start 98.806 57.531) (end 96.901 54.356) (width 1) (layer F.Cu) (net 3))
 (segment (start 96.901 54.356) (end 96.901 52.324) (width 1) (layer F.Cu) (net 3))
 (segment (start 96.901 52.324) (end 94.361 49.784) (width 1) (layer F.Cu) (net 3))
 (segment (start 94.361 49.784) (end 90.805 49.784) (width 1) (layer F.Cu) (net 3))
 (segment (start 80.48752 70.70852) (end 81.915 72.39) (width 1) (layer F.Cu) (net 3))
 (segment (start 80.34782 70.70852) (end 80.48752 70.70852) (width 0.25) (layer F.Cu) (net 3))
 (segment (start 101.219 54.89702) (end 101.219 57.404) (width 1) (layer F.Cu) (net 4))
 (segment (start 101.219 57.404) (end 106.045 57.404) (width 1) (layer F.Cu) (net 4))
 (segment (start 100.33 74.168) (end 100.33 74.041) (width 1) (layer F.Cu) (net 12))
 (segment (start 100.33 74.041) (end 101.727 72.644) (width 1) (layer F.Cu) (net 12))
 (segment (start 104.267 65.024) (end 106.045 65.024) (width 0.5) (layer F.Cu) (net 12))
 (segment (start 101.727 65.405) (end 104.267 65.024) (width 0.5) (layer F.Cu) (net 12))
 (segment (start 101.727 71.247) (end 101.727 65.405) (width 0.5) (layer F.Cu) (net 12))
 (segment (start 101.727 72.644) (end 101.727 71.247) (width 0.5) (layer F.Cu) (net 12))
 (segment (start 67.8942 74.168) (end 100.33 74.168) (width 0.5) (layer F.Cu) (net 12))
 (segment (start 67.9196 74.1426) (end 67.8942 74.168) (width 0.5) (layer F.Cu) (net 12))
 (segment (start 67.9196 70.71614) (end 67.9196 74.1426) (width 0.5) (layer F.Cu) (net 12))
 (segment (start 89.535 70.104) (end 90.805 70.104) (width 0.5) (layer F.Cu) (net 15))
 (segment (start 67.96786 60.452) (end 67.96786 60.47486) (width 0.5) (layer F.Cu) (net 15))
 (segment (start 67.96786 54.02326) (end 67.96786 60.452) (width 0.5) (layer F.Cu) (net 15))
 (segment (start 67.96786 61.74486) (end 68.961 62.738) (width 0.5) (layer F.Cu) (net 15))
 (segment (start 68.961 62.738) (end 72.009 62.738) (width 0.5) (layer F.Cu) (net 15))
 (segment (start 72.009 62.738) (end 75.311 66.04) (width 0.5) (layer F.Cu) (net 15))
 (segment (start 75.311 66.04) (end 80.899 66.04) (width 0.5) (layer F.Cu) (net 15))
 (segment (start 80.899 66.04) (end 84.963 70.104) (width 0.5) (layer F.Cu) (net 15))
 (segment (start 84.963 70.104) (end 90.805 70.104) (width 0.5) (layer F.Cu) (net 15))
 (segment (start 67.96786 60.452) (end 67.96786 61.74486) (width 0.5) (layer F.Cu) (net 15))
 (segment (start 90.297 67.056) (end 90.805 67.564) (width 0.25) (layer F.Cu) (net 16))
 (segment (start 72.76592 60.70092) (end 75.311 63.246) (width 0.5) (layer F.Cu) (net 16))
 (segment (start 75.311 63.246) (end 83.185 63.246) (width 0.5) (layer F.Cu) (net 16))
 (segment (start 83.185 63.246) (end 87.503 67.564) (width 0.5) (layer F.Cu) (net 16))
 (segment (start 87.503 67.564) (end 90.805 67.564) (width 0.5) (layer F.Cu) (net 16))
 (segment (start 69.97192 60.19292) (end 69.97192 60.70092) (width 0.5) (layer F.Cu) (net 16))
 (segment (start 69.97192 54.01564) (end 69.97192 60.19292) (width 0.5) (layer F.Cu) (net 16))
 (segment (start 69.97192 60.70092) (end 72.76592 60.70092) (width 0.5) (layer F.Cu) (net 16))
 (segment (start 87.757 65.024) (end 83.693 60.96) (width 0.5) (layer F.Cu) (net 17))
 (segment (start 83.693 60.96) (end 75.565 60.96) (width 0.5) (layer F.Cu) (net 17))
 (segment (start 75.565 60.96) (end 71.97598 57.37098) (width 0.5) (layer F.Cu) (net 17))
 (segment (start 71.97598 57.37098) (end 71.97598 54.01818) (width 0.5) (layer F.Cu) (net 17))
 (segment (start 90.805 65.024) (end 87.757 65.024) (width 0.5) (layer F.Cu) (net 17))
 (segment (start 74.12482 54.03088) (end 74.168 54.07406) (width 0.5) (layer F.Cu) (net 18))
 (segment (start 74.168 54.07406) (end 74.168 57.277) (width 0.5) (layer F.Cu) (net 18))
 (segment (start 74.168 57.277) (end 74.295 57.277) (width 0.5) (layer F.Cu) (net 18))
 (segment (start 74.295 57.277) (end 74.295 57.404) (width 0.5) (layer F.Cu) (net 18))
 (segment (start 74.295 57.404) (end 76.2 59.309) (width 0.5) (layer F.Cu) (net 18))
 (segment (start 76.2 59.309) (end 84.709 59.309) (width 0.5) (layer F.Cu) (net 18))
 (segment (start 84.709 59.309) (end 87.884 62.484) (width 0.5) (layer F.Cu) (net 18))
 (segment (start 87.884 62.484) (end 90.805 62.484) (width 0.5) (layer F.Cu) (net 18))
 (via (at 78.232 51.435) (size 0.6) (layers F.Cu B.Cu) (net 30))
 (segment (start 78.24216 54.02834) (end 78.232 53.76418) (width 0.25) (layer F.Cu) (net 30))
 (segment (start 78.232 53.76418) (end 78.232 51.435) (width 0.5) (layer F.Cu) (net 30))
 (segment (start 56.642 41.021) (end 56.515 40.894) (width 0.5) (layer F.Cu) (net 30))
 (segment (start 56.642 73.914) (end 56.642 41.021) (width 0.5) (layer F.Cu) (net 30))
 (segment (start 58.166 73.914) (end 56.642 73.914) (width 0.5) (layer F.Cu) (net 30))
 (segment (start 58.166 39.243) (end 58.166 73.914) (width 0.5) (layer F.Cu) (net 30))
 (segment (start 60.198 39.243) (end 58.166 39.243) (width 0.5) (layer F.Cu) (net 30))
 (segment (start 60.198 73.914) (end 60.198 39.243) (width 0.5) (layer F.Cu) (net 30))
 (segment (start 61.468 73.914) (end 60.198 73.914) (width 0.5) (layer F.Cu) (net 30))
 (segment (start 61.468 39.116) (end 61.468 73.914) (width 0.5) (layer F.Cu) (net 30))
 (segment (start 63.373 39.116) (end 61.468 39.116) (width 0.5) (layer F.Cu) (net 30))
 (segment (start 63.373 51.435) (end 63.373 39.116) (width 0.5) (layer F.Cu) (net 30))
 (segment (start 78.232 51.435) (end 63.373 51.435) (width 0.5) (layer F.Cu) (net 30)))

